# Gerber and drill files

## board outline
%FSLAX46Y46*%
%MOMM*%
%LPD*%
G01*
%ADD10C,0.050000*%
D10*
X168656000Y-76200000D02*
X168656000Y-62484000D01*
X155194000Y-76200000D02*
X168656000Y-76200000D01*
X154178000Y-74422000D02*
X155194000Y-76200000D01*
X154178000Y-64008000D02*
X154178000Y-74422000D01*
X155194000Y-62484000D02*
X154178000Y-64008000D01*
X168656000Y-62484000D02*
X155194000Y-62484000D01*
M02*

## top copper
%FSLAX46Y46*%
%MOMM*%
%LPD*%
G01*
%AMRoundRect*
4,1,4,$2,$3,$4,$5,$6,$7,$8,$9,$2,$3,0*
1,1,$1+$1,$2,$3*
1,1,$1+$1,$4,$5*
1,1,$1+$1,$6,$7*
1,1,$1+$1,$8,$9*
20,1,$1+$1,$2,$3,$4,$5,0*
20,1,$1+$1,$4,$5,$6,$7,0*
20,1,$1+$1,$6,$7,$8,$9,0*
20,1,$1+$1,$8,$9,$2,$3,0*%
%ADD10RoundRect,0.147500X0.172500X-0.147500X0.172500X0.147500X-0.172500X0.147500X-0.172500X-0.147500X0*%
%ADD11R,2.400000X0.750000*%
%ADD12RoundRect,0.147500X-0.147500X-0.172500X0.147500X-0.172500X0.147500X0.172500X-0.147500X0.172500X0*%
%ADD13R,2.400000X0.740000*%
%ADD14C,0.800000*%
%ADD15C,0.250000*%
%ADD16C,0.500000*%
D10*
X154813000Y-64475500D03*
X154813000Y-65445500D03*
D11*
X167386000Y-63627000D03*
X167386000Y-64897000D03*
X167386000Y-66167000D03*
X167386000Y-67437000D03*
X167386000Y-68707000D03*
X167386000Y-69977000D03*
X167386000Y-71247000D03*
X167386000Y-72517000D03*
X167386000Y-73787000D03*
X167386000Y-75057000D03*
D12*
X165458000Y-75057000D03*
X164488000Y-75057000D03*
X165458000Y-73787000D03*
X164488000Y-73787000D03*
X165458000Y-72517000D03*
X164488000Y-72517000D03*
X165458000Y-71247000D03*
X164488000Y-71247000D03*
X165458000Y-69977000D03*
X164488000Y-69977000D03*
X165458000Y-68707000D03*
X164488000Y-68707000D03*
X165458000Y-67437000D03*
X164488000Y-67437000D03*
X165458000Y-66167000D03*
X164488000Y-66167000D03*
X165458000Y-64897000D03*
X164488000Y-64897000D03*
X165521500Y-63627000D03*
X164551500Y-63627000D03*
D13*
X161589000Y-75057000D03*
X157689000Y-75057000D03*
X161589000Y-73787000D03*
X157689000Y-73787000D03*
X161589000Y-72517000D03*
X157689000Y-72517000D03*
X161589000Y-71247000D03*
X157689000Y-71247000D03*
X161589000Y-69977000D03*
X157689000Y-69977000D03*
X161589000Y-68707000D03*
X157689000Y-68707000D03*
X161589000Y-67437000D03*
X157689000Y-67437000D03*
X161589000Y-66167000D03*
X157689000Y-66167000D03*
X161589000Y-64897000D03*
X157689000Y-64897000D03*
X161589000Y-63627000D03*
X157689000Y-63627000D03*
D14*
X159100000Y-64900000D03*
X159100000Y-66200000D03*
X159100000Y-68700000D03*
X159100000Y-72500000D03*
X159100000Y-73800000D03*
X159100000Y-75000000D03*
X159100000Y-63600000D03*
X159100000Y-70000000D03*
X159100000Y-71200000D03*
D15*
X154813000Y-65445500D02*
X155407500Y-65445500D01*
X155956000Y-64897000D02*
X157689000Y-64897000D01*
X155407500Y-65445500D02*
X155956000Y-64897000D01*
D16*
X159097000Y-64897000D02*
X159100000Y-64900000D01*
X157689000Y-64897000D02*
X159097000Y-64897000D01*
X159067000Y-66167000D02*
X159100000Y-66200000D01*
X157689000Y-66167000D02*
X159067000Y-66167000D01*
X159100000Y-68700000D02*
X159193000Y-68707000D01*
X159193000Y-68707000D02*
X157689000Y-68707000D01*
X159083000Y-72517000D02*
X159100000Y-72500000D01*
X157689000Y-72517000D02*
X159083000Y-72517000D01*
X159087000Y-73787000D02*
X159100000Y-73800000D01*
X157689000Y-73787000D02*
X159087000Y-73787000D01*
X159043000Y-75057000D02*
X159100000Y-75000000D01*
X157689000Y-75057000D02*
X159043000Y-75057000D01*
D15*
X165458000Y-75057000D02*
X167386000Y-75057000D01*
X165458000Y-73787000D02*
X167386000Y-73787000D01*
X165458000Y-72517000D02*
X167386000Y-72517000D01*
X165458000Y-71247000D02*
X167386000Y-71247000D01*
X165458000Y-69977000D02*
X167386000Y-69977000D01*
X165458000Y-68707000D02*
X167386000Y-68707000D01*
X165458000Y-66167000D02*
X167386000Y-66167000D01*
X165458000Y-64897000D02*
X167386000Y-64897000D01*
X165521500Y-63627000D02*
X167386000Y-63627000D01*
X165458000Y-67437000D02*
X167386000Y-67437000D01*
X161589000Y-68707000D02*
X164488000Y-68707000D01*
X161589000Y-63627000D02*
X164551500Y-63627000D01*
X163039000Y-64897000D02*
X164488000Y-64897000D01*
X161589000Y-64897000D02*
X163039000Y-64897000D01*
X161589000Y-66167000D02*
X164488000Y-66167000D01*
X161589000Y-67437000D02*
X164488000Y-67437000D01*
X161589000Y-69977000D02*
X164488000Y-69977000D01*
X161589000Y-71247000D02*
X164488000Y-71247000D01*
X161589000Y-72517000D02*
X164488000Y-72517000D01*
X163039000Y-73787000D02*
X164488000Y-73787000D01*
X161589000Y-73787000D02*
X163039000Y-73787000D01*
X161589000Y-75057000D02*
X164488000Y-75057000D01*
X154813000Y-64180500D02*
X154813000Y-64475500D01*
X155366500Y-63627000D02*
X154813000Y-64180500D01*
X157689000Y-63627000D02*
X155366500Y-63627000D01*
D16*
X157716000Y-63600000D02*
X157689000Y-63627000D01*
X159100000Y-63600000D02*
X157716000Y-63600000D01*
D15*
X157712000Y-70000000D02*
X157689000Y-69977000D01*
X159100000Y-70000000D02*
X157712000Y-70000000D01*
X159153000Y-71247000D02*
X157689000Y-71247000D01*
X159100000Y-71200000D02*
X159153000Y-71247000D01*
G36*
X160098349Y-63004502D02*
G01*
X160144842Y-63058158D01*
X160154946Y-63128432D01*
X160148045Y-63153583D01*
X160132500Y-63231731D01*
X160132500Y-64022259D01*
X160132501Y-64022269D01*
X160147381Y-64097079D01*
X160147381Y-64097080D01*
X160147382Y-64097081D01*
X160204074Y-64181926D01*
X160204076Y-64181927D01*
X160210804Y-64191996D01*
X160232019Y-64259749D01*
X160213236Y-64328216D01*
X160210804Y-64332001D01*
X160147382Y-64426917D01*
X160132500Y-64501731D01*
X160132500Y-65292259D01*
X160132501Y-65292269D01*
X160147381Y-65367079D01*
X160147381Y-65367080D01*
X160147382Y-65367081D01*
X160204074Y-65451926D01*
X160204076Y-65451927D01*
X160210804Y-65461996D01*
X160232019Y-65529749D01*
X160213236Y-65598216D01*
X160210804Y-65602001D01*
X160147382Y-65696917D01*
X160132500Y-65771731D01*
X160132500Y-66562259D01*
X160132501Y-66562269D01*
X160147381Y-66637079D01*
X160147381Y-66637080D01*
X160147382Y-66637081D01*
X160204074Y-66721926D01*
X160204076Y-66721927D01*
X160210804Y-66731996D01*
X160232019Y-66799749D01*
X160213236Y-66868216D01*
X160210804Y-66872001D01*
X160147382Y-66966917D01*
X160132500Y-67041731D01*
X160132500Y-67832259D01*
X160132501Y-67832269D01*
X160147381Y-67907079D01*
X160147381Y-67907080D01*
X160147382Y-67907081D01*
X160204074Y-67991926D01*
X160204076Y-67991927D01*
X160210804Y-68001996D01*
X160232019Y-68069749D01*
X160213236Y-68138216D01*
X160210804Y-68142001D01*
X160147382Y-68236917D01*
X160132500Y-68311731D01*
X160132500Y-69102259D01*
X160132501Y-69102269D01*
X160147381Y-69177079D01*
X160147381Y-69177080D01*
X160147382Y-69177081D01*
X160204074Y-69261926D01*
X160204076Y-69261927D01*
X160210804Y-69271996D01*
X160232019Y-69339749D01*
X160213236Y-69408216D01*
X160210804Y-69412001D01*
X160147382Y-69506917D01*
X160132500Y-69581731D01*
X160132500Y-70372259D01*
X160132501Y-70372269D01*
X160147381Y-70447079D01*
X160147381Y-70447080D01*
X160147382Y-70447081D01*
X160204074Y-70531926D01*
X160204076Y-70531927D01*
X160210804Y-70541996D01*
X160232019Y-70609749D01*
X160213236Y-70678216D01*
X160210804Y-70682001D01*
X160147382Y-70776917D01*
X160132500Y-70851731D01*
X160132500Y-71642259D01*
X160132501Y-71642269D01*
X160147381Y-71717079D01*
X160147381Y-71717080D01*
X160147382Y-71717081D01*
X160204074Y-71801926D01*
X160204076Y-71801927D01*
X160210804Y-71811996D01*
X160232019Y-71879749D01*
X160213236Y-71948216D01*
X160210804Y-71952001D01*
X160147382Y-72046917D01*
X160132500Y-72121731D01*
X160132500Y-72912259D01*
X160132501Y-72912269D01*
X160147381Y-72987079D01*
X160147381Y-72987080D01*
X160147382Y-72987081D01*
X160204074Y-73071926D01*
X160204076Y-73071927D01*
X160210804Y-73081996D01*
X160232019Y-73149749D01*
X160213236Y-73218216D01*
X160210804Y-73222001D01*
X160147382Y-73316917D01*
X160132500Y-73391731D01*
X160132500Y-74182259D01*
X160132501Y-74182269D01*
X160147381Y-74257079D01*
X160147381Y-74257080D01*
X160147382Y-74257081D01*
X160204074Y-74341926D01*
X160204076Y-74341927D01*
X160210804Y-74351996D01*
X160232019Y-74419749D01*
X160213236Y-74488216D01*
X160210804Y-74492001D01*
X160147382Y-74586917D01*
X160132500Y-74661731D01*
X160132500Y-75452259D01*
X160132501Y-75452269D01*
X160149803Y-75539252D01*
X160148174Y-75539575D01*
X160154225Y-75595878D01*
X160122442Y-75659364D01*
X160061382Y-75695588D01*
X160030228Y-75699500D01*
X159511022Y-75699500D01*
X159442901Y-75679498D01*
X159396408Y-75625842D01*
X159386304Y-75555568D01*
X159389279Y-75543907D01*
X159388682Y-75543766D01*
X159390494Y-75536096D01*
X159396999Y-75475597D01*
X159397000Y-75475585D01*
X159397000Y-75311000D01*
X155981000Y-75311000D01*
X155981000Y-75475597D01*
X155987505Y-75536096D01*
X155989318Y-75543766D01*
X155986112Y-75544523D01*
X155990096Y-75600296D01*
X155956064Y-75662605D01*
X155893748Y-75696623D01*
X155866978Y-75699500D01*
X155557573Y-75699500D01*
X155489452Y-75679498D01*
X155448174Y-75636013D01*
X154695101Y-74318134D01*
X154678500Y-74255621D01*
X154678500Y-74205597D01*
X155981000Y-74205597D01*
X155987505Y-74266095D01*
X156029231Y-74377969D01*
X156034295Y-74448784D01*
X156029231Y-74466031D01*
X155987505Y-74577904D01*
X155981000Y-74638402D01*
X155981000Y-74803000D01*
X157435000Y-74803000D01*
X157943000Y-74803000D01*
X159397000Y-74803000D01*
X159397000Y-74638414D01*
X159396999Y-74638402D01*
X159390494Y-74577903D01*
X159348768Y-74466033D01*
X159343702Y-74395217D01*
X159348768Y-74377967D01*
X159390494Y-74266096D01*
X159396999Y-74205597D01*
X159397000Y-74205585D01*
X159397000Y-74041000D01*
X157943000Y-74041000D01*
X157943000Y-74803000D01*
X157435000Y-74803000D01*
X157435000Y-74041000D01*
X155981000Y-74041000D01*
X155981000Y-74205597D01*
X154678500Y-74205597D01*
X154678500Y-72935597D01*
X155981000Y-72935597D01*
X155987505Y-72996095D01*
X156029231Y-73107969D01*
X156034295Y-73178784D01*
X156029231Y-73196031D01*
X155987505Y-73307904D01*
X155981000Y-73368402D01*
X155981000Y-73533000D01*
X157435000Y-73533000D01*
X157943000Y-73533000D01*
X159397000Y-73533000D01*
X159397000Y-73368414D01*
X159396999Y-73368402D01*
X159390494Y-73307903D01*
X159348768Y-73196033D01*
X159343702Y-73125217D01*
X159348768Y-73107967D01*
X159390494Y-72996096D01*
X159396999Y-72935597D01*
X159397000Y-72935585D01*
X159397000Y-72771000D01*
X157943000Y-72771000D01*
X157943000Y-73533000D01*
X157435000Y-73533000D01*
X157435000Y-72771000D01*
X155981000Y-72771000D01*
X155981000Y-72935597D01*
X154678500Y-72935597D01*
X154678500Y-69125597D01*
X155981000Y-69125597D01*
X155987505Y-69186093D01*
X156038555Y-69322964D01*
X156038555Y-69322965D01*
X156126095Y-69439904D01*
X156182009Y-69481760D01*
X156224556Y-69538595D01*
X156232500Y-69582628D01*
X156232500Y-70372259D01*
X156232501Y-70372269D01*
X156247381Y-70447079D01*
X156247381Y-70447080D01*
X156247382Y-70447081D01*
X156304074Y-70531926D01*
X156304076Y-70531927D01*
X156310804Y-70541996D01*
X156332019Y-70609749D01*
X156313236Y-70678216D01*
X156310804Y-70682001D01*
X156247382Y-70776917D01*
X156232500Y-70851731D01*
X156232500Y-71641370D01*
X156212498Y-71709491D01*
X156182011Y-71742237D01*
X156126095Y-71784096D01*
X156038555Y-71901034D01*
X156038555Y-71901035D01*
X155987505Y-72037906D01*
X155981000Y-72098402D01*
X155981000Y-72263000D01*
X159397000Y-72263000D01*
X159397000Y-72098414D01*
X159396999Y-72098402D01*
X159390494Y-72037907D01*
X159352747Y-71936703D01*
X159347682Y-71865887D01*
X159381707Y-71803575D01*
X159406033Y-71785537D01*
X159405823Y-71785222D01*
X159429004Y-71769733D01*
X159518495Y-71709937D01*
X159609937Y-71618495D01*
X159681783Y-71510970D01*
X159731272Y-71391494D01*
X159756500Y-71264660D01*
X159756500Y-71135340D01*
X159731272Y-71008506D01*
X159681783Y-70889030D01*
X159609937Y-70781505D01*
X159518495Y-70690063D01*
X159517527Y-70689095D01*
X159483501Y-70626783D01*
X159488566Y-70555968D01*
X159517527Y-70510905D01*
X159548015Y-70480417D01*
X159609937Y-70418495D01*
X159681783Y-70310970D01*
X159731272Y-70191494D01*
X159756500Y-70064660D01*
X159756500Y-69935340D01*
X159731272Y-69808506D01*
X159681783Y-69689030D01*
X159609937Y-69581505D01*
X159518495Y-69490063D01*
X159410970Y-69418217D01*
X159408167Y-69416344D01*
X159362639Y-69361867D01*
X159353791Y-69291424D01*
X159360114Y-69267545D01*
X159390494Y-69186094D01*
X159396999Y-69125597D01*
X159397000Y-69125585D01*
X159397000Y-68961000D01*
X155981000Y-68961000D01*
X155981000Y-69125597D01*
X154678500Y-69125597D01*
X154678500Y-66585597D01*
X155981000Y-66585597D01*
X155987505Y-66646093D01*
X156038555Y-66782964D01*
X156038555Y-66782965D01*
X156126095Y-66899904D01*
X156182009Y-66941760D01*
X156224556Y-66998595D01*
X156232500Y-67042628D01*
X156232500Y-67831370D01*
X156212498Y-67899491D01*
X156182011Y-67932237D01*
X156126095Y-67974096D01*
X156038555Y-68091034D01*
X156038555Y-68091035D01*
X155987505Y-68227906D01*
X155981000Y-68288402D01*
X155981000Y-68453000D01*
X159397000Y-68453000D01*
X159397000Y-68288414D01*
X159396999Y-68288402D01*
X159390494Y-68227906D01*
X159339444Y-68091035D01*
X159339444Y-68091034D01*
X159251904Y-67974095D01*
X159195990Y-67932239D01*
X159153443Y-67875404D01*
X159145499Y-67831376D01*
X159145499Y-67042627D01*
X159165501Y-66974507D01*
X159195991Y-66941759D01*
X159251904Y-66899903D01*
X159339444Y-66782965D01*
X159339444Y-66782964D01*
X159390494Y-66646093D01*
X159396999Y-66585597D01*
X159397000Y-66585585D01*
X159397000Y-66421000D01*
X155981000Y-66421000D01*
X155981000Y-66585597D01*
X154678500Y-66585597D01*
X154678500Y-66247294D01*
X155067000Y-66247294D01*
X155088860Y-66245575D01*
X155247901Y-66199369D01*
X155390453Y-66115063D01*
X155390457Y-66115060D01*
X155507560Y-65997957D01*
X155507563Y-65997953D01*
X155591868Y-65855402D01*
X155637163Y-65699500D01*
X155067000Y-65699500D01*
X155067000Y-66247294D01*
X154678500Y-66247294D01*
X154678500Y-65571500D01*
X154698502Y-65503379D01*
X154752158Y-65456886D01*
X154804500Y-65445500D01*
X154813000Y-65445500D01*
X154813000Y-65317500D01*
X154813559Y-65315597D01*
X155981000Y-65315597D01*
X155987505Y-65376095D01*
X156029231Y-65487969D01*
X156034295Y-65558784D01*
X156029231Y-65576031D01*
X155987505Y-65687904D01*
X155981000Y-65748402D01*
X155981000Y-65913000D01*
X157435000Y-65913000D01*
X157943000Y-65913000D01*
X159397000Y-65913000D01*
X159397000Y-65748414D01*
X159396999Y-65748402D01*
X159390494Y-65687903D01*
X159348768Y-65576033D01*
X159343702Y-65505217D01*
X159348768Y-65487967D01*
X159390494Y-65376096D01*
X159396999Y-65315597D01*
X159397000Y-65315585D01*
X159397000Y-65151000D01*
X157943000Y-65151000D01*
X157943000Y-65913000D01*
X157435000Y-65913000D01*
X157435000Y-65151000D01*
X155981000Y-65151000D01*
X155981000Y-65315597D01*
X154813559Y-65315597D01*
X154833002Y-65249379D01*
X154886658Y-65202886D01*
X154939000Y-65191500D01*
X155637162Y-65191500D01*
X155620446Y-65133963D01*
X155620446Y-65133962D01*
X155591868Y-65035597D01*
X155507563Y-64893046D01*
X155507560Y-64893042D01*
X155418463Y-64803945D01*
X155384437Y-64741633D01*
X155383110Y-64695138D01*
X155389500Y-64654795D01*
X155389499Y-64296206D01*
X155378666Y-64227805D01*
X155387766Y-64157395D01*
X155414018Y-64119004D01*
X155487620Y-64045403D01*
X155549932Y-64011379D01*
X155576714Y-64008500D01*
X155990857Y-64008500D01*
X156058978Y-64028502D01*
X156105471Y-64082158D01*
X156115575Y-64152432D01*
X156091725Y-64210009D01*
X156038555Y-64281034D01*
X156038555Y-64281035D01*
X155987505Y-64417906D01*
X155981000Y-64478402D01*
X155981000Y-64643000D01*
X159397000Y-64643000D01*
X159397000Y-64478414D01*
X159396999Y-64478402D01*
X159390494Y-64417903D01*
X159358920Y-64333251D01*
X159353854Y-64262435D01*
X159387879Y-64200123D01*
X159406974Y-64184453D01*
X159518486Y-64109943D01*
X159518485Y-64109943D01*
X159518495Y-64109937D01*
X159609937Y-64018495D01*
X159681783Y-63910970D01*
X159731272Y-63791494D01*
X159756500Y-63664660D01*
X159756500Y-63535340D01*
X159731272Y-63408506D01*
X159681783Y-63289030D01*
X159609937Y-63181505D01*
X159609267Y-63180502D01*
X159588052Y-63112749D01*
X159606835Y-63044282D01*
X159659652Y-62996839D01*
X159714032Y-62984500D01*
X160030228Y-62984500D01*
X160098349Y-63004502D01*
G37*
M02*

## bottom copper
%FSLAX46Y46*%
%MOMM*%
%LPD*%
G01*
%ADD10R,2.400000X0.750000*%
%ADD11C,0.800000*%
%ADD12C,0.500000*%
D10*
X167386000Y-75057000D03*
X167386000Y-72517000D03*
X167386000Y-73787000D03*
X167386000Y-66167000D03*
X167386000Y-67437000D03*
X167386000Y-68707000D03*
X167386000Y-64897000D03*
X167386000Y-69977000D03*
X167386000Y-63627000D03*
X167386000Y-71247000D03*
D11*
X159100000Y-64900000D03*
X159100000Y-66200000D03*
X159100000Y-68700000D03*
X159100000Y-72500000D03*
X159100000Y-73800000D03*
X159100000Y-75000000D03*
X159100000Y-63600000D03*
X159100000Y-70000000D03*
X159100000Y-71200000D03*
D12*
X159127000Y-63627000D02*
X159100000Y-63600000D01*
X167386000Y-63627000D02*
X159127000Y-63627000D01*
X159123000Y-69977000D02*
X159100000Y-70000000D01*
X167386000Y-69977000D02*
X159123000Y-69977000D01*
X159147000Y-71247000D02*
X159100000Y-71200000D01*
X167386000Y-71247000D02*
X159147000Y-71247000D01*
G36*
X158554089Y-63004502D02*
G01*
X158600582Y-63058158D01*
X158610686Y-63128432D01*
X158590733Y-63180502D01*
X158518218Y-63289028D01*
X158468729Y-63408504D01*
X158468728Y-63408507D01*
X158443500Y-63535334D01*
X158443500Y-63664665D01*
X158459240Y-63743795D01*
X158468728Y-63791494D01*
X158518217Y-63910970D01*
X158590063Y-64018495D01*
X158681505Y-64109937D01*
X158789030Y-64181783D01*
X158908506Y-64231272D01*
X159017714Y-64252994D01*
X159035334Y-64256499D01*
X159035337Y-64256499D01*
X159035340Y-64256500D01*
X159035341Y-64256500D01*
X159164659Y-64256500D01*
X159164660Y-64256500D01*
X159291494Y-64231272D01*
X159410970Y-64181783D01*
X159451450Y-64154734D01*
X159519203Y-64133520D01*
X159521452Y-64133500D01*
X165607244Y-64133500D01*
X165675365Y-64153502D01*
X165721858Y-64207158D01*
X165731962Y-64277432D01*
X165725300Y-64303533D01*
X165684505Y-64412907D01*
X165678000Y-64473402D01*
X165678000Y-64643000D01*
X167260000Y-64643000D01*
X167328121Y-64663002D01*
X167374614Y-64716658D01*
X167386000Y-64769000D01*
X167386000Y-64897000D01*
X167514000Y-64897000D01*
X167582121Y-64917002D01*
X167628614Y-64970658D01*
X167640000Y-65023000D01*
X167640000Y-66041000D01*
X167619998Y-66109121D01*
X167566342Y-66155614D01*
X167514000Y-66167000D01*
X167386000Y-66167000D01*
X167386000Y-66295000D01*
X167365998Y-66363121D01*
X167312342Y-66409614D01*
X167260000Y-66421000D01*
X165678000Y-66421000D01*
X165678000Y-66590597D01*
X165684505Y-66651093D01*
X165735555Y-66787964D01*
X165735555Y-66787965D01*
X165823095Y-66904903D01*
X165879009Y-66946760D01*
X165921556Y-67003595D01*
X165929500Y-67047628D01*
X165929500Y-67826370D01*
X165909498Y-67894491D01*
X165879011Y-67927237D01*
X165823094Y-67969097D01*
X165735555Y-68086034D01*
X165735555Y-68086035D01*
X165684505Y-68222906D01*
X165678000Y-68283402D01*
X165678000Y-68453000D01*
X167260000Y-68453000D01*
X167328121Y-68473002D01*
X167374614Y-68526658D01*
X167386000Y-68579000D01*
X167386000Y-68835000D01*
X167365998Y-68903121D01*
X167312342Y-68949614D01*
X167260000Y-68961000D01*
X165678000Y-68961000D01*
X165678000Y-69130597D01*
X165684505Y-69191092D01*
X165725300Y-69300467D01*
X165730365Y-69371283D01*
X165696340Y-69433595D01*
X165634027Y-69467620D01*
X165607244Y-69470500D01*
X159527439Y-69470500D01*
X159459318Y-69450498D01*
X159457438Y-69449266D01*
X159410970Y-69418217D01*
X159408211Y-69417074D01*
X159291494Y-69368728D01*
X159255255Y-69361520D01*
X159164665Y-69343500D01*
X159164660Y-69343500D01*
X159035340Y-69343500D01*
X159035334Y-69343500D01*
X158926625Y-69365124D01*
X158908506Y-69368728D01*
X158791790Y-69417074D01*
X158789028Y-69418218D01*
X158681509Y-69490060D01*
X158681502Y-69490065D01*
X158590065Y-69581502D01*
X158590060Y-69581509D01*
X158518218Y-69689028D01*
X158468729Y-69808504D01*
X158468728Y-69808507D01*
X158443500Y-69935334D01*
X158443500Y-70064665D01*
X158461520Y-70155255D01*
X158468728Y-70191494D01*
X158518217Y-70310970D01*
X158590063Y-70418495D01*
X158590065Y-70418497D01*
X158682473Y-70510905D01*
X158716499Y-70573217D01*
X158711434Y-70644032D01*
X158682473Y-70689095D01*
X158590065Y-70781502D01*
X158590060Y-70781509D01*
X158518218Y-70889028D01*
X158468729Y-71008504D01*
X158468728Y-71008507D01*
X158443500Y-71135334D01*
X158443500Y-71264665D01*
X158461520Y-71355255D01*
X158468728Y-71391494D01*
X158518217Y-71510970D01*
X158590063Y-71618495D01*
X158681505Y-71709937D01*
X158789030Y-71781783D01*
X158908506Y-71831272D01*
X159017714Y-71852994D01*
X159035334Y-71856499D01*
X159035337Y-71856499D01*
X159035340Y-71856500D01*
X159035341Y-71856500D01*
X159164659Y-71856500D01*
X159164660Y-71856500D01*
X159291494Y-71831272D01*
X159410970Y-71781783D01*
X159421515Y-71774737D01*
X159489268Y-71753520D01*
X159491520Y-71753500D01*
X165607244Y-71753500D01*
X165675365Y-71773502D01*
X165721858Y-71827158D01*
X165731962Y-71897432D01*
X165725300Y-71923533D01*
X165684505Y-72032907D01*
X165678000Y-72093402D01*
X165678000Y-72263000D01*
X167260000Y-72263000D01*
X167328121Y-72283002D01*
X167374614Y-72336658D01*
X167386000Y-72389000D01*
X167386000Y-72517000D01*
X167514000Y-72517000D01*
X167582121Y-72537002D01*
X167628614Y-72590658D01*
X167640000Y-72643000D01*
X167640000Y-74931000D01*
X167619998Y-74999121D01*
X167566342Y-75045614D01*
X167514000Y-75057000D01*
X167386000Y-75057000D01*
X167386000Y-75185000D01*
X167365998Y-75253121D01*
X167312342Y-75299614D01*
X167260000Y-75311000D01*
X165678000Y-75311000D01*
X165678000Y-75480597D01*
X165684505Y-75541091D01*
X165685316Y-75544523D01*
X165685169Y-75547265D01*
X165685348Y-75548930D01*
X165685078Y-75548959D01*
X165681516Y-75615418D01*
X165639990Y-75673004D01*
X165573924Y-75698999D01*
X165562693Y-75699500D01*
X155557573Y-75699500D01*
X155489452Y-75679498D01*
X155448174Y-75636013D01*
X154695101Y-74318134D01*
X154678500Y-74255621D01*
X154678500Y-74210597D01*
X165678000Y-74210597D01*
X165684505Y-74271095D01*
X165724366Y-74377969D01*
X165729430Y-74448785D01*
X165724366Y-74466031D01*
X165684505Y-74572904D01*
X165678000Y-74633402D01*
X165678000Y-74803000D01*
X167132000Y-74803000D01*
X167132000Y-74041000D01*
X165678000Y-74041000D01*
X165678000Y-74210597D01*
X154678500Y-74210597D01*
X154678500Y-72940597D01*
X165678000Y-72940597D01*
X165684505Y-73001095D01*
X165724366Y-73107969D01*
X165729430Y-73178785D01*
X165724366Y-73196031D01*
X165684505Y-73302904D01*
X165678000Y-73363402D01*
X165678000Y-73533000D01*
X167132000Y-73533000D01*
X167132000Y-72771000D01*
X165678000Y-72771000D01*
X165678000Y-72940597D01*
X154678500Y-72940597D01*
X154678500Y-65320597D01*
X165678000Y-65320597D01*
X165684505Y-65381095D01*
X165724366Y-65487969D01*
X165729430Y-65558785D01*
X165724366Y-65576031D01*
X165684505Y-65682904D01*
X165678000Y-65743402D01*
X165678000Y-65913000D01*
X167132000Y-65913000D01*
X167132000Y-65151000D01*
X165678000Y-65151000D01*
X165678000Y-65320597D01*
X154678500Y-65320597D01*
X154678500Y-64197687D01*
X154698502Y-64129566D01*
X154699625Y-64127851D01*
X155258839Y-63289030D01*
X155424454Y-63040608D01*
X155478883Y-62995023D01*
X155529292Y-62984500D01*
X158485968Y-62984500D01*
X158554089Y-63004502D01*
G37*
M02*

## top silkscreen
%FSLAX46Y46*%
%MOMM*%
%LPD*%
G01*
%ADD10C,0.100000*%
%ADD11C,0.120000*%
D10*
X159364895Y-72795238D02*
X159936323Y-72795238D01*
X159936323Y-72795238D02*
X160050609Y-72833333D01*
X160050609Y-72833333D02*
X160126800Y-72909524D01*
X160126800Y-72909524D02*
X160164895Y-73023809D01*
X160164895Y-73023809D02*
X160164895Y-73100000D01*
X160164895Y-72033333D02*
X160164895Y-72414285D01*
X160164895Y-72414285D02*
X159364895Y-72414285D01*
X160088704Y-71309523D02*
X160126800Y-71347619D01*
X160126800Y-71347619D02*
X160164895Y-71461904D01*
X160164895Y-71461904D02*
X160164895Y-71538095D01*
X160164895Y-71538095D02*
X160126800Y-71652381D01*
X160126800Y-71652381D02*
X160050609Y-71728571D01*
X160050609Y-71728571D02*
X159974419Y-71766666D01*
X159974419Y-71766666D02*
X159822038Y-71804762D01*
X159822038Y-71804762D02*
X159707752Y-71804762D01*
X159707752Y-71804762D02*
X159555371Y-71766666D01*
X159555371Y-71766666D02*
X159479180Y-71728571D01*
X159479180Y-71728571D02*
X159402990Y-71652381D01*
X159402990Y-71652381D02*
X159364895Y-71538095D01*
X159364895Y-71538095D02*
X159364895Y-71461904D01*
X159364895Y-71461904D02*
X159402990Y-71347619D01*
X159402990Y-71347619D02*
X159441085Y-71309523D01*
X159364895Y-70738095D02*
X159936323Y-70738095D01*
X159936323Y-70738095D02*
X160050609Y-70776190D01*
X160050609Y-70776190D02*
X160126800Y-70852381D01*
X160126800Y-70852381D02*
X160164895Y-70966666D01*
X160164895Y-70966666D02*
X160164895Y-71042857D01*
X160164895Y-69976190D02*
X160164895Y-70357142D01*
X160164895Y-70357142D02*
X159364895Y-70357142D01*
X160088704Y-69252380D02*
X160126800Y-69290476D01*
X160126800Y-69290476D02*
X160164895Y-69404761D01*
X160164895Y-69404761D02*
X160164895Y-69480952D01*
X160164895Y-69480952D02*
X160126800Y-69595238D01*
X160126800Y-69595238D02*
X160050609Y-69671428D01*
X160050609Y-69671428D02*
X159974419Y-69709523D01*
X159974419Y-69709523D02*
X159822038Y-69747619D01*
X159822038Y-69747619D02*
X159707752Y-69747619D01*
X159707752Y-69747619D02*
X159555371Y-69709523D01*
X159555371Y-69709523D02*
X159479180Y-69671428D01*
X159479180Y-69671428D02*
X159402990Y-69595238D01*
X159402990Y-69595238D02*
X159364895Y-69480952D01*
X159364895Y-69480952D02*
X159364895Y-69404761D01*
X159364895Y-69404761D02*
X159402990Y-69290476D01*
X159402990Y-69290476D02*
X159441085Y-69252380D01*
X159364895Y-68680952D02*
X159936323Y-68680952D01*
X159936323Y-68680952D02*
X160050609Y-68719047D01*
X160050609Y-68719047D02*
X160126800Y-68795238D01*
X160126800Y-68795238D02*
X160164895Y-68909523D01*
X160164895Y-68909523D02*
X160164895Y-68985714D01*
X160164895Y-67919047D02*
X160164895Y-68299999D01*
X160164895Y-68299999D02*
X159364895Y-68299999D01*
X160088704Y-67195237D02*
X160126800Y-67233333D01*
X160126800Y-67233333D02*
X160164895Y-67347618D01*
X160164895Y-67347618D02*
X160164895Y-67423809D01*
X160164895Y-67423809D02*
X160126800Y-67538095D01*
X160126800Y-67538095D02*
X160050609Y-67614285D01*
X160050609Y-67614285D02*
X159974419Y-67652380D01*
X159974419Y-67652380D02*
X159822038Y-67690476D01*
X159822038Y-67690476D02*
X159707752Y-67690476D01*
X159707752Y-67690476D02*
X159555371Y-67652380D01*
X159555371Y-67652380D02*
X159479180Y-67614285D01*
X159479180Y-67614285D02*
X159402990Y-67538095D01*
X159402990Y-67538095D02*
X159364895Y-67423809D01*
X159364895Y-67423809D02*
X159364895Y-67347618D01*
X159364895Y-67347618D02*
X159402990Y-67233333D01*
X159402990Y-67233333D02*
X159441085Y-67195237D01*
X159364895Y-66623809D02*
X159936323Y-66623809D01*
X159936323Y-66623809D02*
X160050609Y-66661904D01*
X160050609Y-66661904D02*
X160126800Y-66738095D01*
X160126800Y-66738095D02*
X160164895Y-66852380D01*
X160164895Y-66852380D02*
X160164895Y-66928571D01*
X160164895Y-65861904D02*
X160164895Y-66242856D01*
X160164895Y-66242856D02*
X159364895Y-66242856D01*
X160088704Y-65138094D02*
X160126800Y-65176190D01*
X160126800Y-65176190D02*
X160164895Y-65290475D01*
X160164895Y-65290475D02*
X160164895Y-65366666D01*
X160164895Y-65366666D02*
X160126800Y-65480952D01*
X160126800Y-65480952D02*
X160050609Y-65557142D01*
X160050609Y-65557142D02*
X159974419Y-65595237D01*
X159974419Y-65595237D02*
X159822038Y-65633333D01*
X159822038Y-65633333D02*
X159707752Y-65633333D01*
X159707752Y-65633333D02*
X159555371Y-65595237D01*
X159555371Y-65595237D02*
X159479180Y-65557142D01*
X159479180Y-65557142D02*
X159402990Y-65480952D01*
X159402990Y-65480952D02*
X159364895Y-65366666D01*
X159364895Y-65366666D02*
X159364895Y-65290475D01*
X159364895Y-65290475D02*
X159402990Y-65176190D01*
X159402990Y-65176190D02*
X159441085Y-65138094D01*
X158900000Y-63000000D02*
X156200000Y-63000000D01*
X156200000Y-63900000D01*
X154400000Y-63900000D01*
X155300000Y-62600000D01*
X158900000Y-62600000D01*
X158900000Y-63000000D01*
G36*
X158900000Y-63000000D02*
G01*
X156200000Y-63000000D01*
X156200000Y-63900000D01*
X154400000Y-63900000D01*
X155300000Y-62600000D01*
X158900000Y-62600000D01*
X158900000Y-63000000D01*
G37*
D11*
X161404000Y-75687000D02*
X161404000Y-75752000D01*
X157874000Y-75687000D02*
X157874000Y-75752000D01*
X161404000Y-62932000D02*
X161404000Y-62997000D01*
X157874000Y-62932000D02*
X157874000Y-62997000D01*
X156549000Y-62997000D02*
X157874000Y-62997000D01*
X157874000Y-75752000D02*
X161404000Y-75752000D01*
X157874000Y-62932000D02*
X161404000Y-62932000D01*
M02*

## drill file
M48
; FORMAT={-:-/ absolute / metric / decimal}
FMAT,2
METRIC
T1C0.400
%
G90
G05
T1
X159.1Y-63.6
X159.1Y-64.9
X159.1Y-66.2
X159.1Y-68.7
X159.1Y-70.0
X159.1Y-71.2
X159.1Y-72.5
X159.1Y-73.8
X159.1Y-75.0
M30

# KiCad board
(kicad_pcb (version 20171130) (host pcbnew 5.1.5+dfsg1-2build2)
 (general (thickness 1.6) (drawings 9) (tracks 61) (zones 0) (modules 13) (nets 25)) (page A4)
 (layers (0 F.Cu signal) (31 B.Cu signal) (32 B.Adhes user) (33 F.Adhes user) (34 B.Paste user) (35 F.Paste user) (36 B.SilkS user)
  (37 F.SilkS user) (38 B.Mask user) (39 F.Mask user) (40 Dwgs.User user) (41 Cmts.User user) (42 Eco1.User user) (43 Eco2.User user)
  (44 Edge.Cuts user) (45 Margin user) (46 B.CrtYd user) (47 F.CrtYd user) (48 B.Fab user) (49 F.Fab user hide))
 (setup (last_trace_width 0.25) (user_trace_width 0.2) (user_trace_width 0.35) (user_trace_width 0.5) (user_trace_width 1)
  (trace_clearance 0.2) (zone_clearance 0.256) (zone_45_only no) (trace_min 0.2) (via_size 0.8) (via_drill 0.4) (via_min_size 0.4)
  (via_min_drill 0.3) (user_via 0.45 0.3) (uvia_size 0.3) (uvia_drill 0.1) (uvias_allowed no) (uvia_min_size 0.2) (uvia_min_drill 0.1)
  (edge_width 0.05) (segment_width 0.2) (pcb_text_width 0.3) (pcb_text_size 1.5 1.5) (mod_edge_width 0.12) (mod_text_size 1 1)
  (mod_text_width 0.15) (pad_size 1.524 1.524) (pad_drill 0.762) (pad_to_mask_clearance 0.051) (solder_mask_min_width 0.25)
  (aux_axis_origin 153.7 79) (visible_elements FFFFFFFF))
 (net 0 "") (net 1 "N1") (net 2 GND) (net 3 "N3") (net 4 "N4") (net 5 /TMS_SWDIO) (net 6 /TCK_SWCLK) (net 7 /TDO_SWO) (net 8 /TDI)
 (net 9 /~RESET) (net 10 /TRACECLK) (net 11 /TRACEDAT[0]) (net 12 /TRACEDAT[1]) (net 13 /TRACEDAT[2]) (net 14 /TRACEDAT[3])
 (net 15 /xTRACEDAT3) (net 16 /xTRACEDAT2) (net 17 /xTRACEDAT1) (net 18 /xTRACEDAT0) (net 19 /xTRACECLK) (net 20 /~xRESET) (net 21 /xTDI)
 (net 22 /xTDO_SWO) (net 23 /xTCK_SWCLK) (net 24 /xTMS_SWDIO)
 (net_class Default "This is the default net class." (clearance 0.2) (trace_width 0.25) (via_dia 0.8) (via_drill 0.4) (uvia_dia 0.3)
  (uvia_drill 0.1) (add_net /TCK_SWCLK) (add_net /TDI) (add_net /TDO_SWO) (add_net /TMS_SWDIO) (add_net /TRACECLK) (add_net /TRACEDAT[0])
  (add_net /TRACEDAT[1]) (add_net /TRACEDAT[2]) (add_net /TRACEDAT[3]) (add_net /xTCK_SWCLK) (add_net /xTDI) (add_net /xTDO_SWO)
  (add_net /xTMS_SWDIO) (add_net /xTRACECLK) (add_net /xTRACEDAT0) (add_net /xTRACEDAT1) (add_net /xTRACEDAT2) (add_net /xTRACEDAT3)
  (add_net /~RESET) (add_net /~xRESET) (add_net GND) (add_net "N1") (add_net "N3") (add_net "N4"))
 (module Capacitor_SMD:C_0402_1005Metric (layer F.Cu) (at 154.813 64.9605 90)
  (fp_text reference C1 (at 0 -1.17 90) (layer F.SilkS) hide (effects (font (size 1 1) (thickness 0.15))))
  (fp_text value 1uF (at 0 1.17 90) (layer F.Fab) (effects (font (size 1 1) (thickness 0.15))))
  (pad 2 smd roundrect (at 0.485 0 90) (size 0.59 0.64) (layers F.Cu F.Paste F.Mask) (roundrect_rratio 0.25) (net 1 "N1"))
  (pad 1 smd roundrect (at -0.485 0 90) (size 0.59 0.64) (layers F.Cu F.Paste F.Mask) (roundrect_rratio 0.25) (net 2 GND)))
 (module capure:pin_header (layer F.Cu) (at 167.386 75.057)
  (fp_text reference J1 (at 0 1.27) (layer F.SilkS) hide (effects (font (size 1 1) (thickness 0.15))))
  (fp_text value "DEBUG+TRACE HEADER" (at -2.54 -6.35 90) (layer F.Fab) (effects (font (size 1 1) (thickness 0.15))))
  (pad 19 smd rect (at 0 0) (size 2.4 0.75) (layers B.Cu B.Paste B.Mask) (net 2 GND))
  (pad 15 smd rect (at 0 -2.54) (size 2.4 0.75) (layers B.Cu B.Paste B.Mask) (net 2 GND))
  (pad 17 smd rect (at 0 -1.27) (size 2.4 0.75) (layers B.Cu B.Paste B.Mask) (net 2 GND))
  (pad 5 smd rect (at 0 -8.89) (size 2.4 0.75) (layers B.Cu B.Paste B.Mask) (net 2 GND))
  (pad 7 smd rect (at 0 -7.62) (size 2.4 0.75) (layers B.Cu B.Paste B.Mask))
  (pad 9 smd rect (at 0 -6.35) (size 2.4 0.75) (layers B.Cu B.Paste B.Mask) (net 2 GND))
  (pad 3 smd rect (at 0 -10.16) (size 2.4 0.75) (layers B.Cu B.Paste B.Mask) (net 2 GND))
  (pad 11 smd rect (at 0 -5.08) (size 2.4 0.75) (layers B.Cu B.Paste B.Mask) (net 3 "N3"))
  (pad 1 smd rect (at 0 -11.43) (size 2.4 0.75) (layers B.Cu B.Paste B.Mask) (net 1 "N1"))
  (pad 13 smd rect (at 0 -3.81) (size 2.4 0.75) (layers B.Cu B.Paste B.Mask) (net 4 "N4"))
  (pad 2 smd rect (at 0 -11.43) (size 2.4 0.75) (layers F.Cu F.Paste F.Mask) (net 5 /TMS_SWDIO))
  (pad 4 smd rect (at 0 -10.16) (size 2.4 0.75) (layers F.Cu F.Paste F.Mask) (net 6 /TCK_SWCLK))
  (pad 6 smd rect (at 0 -8.89) (size 2.4 0.75) (layers F.Cu F.Paste F.Mask) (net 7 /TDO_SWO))
  (pad 8 smd rect (at 0 -7.62) (size 2.4 0.75) (layers F.Cu F.Paste F.Mask) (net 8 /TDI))
  (pad 10 smd rect (at 0 -6.35) (size 2.4 0.75) (layers F.Cu F.Paste F.Mask) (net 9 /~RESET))
  (pad 12 smd rect (at 0 -5.08) (size 2.4 0.75) (layers F.Cu F.Paste F.Mask) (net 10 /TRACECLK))
  (pad 14 smd rect (at 0 -3.81) (size 2.4 0.75) (layers F.Cu F.Paste F.Mask) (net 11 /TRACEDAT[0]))
  (pad 16 smd rect (at 0 -2.54) (size 2.4 0.75) (layers F.Cu F.Paste F.Mask) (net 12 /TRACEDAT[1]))
  (pad 18 smd rect (at 0 -1.27) (size 2.4 0.75) (layers F.Cu F.Paste F.Mask) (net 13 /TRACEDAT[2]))
  (pad 20 smd rect (at 0 0) (size 2.4 0.75) (layers F.Cu F.Paste F.Mask) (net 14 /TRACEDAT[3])))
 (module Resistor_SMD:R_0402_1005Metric (layer F.Cu) (at 164.973 75.057)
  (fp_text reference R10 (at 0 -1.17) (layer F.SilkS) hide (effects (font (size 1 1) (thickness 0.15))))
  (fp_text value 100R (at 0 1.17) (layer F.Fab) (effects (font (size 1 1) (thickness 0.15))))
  (pad 2 smd roundrect (at 0.485 0) (size 0.59 0.64) (layers F.Cu F.Paste F.Mask) (roundrect_rratio 0.25) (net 14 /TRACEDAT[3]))
  (pad 1 smd roundrect (at -0.485 0) (size 0.59 0.64) (layers F.Cu F.Paste F.Mask) (roundrect_rratio 0.25) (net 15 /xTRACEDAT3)))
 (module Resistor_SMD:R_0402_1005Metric (layer F.Cu) (at 164.973 73.787)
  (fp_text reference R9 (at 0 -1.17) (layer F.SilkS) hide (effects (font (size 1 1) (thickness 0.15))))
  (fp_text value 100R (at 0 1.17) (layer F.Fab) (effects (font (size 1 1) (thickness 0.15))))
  (pad 2 smd roundrect (at 0.485 0) (size 0.59 0.64) (layers F.Cu F.Paste F.Mask) (roundrect_rratio 0.25) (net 13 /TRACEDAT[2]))
  (pad 1 smd roundrect (at -0.485 0) (size 0.59 0.64) (layers F.Cu F.Paste F.Mask) (roundrect_rratio 0.25) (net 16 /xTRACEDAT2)))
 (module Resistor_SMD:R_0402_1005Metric (layer F.Cu) (at 164.973 72.517)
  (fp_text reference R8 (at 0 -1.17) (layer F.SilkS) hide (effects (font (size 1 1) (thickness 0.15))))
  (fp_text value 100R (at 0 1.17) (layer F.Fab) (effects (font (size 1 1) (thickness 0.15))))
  (pad 2 smd roundrect (at 0.485 0) (size 0.59 0.64) (layers F.Cu F.Paste F.Mask) (roundrect_rratio 0.25) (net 12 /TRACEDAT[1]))
  (pad 1 smd roundrect (at -0.485 0) (size 0.59 0.64) (layers F.Cu F.Paste F.Mask) (roundrect_rratio 0.25) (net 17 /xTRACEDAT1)))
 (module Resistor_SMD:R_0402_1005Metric (layer F.Cu) (at 164.973 71.247)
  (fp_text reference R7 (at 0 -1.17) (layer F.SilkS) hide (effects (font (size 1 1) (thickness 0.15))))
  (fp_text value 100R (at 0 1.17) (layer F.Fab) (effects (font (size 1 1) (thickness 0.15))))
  (pad 2 smd roundrect (at 0.485 0) (size 0.59 0.64) (layers F.Cu F.Paste F.Mask) (roundrect_rratio 0.25) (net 11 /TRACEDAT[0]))
  (pad 1 smd roundrect (at -0.485 0) (size 0.59 0.64) (layers F.Cu F.Paste F.Mask) (roundrect_rratio 0.25) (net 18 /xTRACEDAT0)))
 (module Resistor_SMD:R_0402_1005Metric (layer F.Cu) (at 164.973 69.977)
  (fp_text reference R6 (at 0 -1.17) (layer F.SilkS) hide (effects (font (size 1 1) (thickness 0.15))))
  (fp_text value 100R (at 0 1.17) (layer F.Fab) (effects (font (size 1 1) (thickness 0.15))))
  (pad 2 smd roundrect (at 0.485 0) (size 0.59 0.64) (layers F.Cu F.Paste F.Mask) (roundrect_rratio 0.25) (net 10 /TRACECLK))
  (pad 1 smd roundrect (at -0.485 0) (size 0.59 0.64) (layers F.Cu F.Paste F.Mask) (roundrect_rratio 0.25) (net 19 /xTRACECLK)))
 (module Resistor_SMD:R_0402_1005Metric (layer F.Cu) (at 164.973 68.707)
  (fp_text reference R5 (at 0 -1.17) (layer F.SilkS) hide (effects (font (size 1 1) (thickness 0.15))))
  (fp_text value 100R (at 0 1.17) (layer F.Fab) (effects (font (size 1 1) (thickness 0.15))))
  (pad 2 smd roundrect (at 0.485 0) (size 0.59 0.64) (layers F.Cu F.Paste F.Mask) (roundrect_rratio 0.25) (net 9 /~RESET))
  (pad 1 smd roundrect (at -0.485 0) (size 0.59 0.64) (layers F.Cu F.Paste F.Mask) (roundrect_rratio 0.25) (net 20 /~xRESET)))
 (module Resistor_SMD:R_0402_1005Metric (layer F.Cu) (at 164.973 67.437)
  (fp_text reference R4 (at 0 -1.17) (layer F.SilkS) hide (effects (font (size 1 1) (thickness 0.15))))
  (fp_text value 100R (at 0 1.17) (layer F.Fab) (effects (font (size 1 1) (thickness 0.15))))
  (pad 2 smd roundrect (at 0.485 0) (size 0.59 0.64) (layers F.Cu F.Paste F.Mask) (roundrect_rratio 0.25) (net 8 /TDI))
  (pad 1 smd roundrect (at -0.485 0) (size 0.59 0.64) (layers F.Cu F.Paste F.Mask) (roundrect_rratio 0.25) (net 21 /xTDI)))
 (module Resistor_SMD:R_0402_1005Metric (layer F.Cu) (at 164.973 66.167)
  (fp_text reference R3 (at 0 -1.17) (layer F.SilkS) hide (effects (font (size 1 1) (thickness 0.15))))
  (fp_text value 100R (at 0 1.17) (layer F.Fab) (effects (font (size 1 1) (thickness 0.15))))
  (pad 2 smd roundrect (at 0.485 0) (size 0.59 0.64) (layers F.Cu F.Paste F.Mask) (roundrect_rratio 0.25) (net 7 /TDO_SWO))
  (pad 1 smd roundrect (at -0.485 0) (size 0.59 0.64) (layers F.Cu F.Paste F.Mask) (roundrect_rratio 0.25) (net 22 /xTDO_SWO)))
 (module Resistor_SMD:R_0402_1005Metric (layer F.Cu) (at 164.973 64.897)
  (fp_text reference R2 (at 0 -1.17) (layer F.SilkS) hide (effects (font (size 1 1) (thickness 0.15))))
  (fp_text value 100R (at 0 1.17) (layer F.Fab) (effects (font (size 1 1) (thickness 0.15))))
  (pad 2 smd roundrect (at 0.485 0) (size 0.59 0.64) (layers F.Cu F.Paste F.Mask) (roundrect_rratio 0.25) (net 6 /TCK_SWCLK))
  (pad 1 smd roundrect (at -0.485 0) (size 0.59 0.64) (layers F.Cu F.Paste F.Mask) (roundrect_rratio 0.25) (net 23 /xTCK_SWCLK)))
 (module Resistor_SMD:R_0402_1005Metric (layer F.Cu) (at 165.0365 63.627)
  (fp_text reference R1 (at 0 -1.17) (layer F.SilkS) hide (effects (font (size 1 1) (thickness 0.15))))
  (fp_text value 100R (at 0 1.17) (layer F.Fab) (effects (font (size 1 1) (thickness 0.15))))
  (pad 2 smd roundrect (at 0.485 0) (size 0.59 0.64) (layers F.Cu F.Paste F.Mask) (roundrect_rratio 0.25) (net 5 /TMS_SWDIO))
  (pad 1 smd roundrect (at -0.485 0) (size 0.59 0.64) (layers F.Cu F.Paste F.Mask) (roundrect_rratio 0.25) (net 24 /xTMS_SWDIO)))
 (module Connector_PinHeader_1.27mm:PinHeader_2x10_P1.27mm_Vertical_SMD (layer F.Cu) (at 159.639 69.342)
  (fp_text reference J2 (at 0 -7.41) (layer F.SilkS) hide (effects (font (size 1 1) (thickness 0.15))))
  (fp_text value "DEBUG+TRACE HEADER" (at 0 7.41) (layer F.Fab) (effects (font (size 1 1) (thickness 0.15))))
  (fp_line (start 1.765 6.345) (end 1.765 6.41) (layer F.SilkS) (width 0.12))
  (fp_line (start -1.765 6.345) (end -1.765 6.41) (layer F.SilkS) (width 0.12))
  (fp_line (start 1.765 -6.41) (end 1.765 -6.345) (layer F.SilkS) (width 0.12))
  (fp_line (start -1.765 -6.41) (end -1.765 -6.345) (layer F.SilkS) (width 0.12))
  (fp_line (start -3.09 -6.345) (end -1.765 -6.345) (layer F.SilkS) (width 0.12))
  (fp_line (start -1.765 6.41) (end 1.765 6.41) (layer F.SilkS) (width 0.12))
  (fp_line (start -1.765 -6.41) (end 1.765 -6.41) (layer F.SilkS) (width 0.12))
  (pad 20 smd rect (at 1.95 5.715) (size 2.4 0.74) (layers F.Cu F.Paste F.Mask) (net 15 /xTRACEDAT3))
  (pad 19 smd rect (at -1.95 5.715) (size 2.4 0.74) (layers F.Cu F.Paste F.Mask) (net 2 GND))
  (pad 18 smd rect (at 1.95 4.445) (size 2.4 0.74) (layers F.Cu F.Paste F.Mask) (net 16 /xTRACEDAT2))
  (pad 17 smd rect (at -1.95 4.445) (size 2.4 0.74) (layers F.Cu F.Paste F.Mask) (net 2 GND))
  (pad 16 smd rect (at 1.95 3.175) (size 2.4 0.74) (layers F.Cu F.Paste F.Mask) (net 17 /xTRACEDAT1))
  (pad 15 smd rect (at -1.95 3.175) (size 2.4 0.74) (layers F.Cu F.Paste F.Mask) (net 2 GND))
  (pad 14 smd rect (at 1.95 1.905) (size 2.4 0.74) (layers F.Cu F.Paste F.Mask) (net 18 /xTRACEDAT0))
  (pad 13 smd rect (at -1.95 1.905) (size 2.4 0.74) (layers F.Cu F.Paste F.Mask) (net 4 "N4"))
  (pad 12 smd rect (at 1.95 0.635) (size 2.4 0.74) (layers F.Cu F.Paste F.Mask) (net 19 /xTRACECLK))
  (pad 11 smd rect (at -1.95 0.635) (size 2.4 0.74) (layers F.Cu F.Paste F.Mask) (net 3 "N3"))
  (pad 10 smd rect (at 1.95 -0.635) (size 2.4 0.74) (layers F.Cu F.Paste F.Mask) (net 20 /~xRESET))
  (pad 9 smd rect (at -1.95 -0.635) (size 2.4 0.74) (layers F.Cu F.Paste F.Mask) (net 2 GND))
  (pad 8 smd rect (at 1.95 -1.905) (size 2.4 0.74) (layers F.Cu F.Paste F.Mask) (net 21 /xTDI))
  (pad 7 smd rect (at -1.95 -1.905) (size 2.4 0.74) (layers F.Cu F.Paste F.Mask))
  (pad 6 smd rect (at 1.95 -3.175) (size 2.4 0.74) (layers F.Cu F.Paste F.Mask) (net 22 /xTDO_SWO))
  (pad 5 smd rect (at -1.95 -3.175) (size 2.4 0.74) (layers F.Cu F.Paste F.Mask) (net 2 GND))
  (pad 4 smd rect (at 1.95 -4.445) (size 2.4 0.74) (layers F.Cu F.Paste F.Mask) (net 23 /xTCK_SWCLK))
  (pad 3 smd rect (at -1.95 -4.445) (size 2.4 0.74) (layers F.Cu F.Paste F.Mask) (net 2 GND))
  (pad 2 smd rect (at 1.95 -5.715) (size 2.4 0.74) (layers F.Cu F.Paste F.Mask) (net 24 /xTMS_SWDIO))
  (pad 1 smd rect (at -1.95 -5.715) (size 2.4 0.74) (layers F.Cu F.Paste F.Mask) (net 1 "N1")))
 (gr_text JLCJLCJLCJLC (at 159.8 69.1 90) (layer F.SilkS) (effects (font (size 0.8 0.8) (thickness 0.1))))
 (gr_poly (pts (xy 158.9 63) (xy 156.2 63) (xy 156.2 63.9) (xy 154.4 63.9) (xy 155.3 62.6) (xy 158.9 62.6)) (layer F.SilkS) (width 0.1))
 (gr_line (start 168.656 76.2) (end 168.656 62.484) (layer Edge.Cuts) (width 0.05))
 (gr_line (start 155.194 76.2) (end 168.656 76.2) (layer Edge.Cuts) (width 0.05))
 (gr_line (start 154.178 74.422) (end 155.194 76.2) (layer Edge.Cuts) (width 0.05))
 (gr_line (start 154.178 64.008) (end 154.178 74.422) (layer Edge.Cuts) (width 0.05))
 (gr_line (start 155.194 62.484) (end 154.178 64.008) (layer Edge.Cuts) (width 0.05))
 (gr_line (start 168.656 62.484) (end 155.194 62.484) (layer Edge.Cuts) (width 0.05))
 (segment (start 154.813 65.4455) (end 155.4075 65.4455) (width 0.25) (layer F.Cu) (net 2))
 (segment (start 155.956 64.897) (end 157.689 64.897) (width 0.25) (layer F.Cu) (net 2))
 (segment (start 155.4075 65.4455) (end 155.956 64.897) (width 0.25) (layer F.Cu) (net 2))
 (via (at 159.1 64.9) (size 0.8) (drill 0.4) (layers F.Cu B.Cu) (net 2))
 (segment (start 159.097 64.897) (end 159.1 64.9) (width 0.5) (layer F.Cu) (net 2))
 (segment (start 157.689 64.897) (end 159.097 64.897) (width 0.5) (layer F.Cu) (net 2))
 (via (at 159.1 66.2) (size 0.8) (drill 0.4) (layers F.Cu B.Cu) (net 2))
 (segment (start 159.067 66.167) (end 159.1 66.2) (width 0.5) (layer F.Cu) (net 2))
 (segment (start 157.689 66.167) (end 159.067 66.167) (width 0.5) (layer F.Cu) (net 2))
 (segment (start 159.1 68.7) (end 159.193 68.707) (width 0.5) (layer F.Cu) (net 2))
 (segment (start 159.193 68.707) (end 157.689 68.707) (width 0.5) (layer F.Cu) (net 2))
 (via (at 159.1 68.7) (size 0.8) (drill 0.4) (layers F.Cu B.Cu) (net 2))
 (via (at 159.1 72.5) (size 0.8) (drill 0.4) (layers F.Cu B.Cu) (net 2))
 (segment (start 159.083 72.517) (end 159.1 72.5) (width 0.5) (layer F.Cu) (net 2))
 (segment (start 157.689 72.517) (end 159.083 72.517) (width 0.5) (layer F.Cu) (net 2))
 (via (at 159.1 73.8) (size 0.8) (drill 0.4) (layers F.Cu B.Cu) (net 2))
 (segment (start 159.087 73.787) (end 159.1 73.8) (width 0.5) (layer F.Cu) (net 2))
 (segment (start 157.689 73.787) (end 159.087 73.787) (width 0.5) (layer F.Cu) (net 2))
 (via (at 159.1 75) (size 0.8) (drill 0.4) (layers F.Cu B.Cu) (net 2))
 (segment (start 159.043 75.057) (end 159.1 75) (width 0.5) (layer F.Cu) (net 2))
 (segment (start 157.689 75.057) (end 159.043 75.057) (width 0.5) (layer F.Cu) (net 2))
 (segment (start 165.458 75.057) (end 167.386 75.057) (width 0.25) (layer F.Cu) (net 14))
 (segment (start 165.458 73.787) (end 167.386 73.787) (width 0.25) (layer F.Cu) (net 13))
 (segment (start 165.458 72.517) (end 167.386 72.517) (width 0.25) (layer F.Cu) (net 12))
 (segment (start 165.458 71.247) (end 167.386 71.247) (width 0.25) (layer F.Cu) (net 11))
 (segment (start 165.458 69.977) (end 167.386 69.977) (width 0.25) (layer F.Cu) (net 10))
 (segment (start 165.458 68.707) (end 167.386 68.707) (width 0.25) (layer F.Cu) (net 9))
 (segment (start 165.458 66.167) (end 167.386 66.167) (width 0.25) (layer F.Cu) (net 7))
 (segment (start 165.458 64.897) (end 167.386 64.897) (width 0.25) (layer F.Cu) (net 6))
 (segment (start 165.5215 63.627) (end 167.386 63.627) (width 0.25) (layer F.Cu) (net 5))
 (segment (start 165.458 67.437) (end 167.386 67.437) (width 0.25) (layer F.Cu) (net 8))
 (segment (start 161.589 68.707) (end 164.488 68.707) (width 0.25) (layer F.Cu) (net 20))
 (segment (start 161.589 63.627) (end 164.5515 63.627) (width 0.25) (layer F.Cu) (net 24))
 (segment (start 163.039 64.897) (end 164.488 64.897) (width 0.25) (layer F.Cu) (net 23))
 (segment (start 161.589 64.897) (end 163.039 64.897) (width 0.25) (layer F.Cu) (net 23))
 (segment (start 161.589 66.167) (end 164.488 66.167) (width 0.25) (layer F.Cu) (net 22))
 (segment (start 161.589 67.437) (end 164.488 67.437) (width 0.25) (layer F.Cu) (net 21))
 (segment (start 161.589 69.977) (end 164.488 69.977) (width 0.25) (layer F.Cu) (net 19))
 (segment (start 161.589 71.247) (end 164.488 71.247) (width 0.25) (layer F.Cu) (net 18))
 (segment (start 161.589 72.517) (end 164.488 72.517) (width 0.25) (layer F.Cu) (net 17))
 (segment (start 163.039 73.787) (end 164.488 73.787) (width 0.25) (layer F.Cu) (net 16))
 (segment (start 161.589 73.787) (end 163.039 73.787) (width 0.25) (layer F.Cu) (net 16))
 (segment (start 161.589 75.057) (end 164.488 75.057) (width 0.25) (layer F.Cu) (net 15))
 (segment (start 154.813 64.1805) (end 154.813 64.4755) (width 0.25) (layer F.Cu) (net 1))
 (segment (start 155.3665 63.627) (end 154.813 64.1805) (width 0.25) (layer F.Cu) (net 1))
 (segment (start 157.689 63.627) (end 155.3665 63.627) (width 0.25) (layer F.Cu) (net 1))
 (via (at 159.1 63.6) (size 0.8) (drill 0.4) (layers F.Cu B.Cu) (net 1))
 (segment (start 159.127 63.627) (end 159.1 63.6) (width 0.5) (layer B.Cu) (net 1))
 (segment (start 167.386 63.627) (end 159.127 63.627) (width 0.5) (layer B.Cu) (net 1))
 (segment (start 157.716 63.6) (end 157.689 63.627) (width 0.5) (layer F.Cu) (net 1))
 (segment (start 159.1 63.6) (end 157.716 63.6) (width 0.5) (layer F.Cu) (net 1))
 (via (at 159.1 70) (size 0.8) (drill 0.4) (layers F.Cu B.Cu) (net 3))
 (segment (start 157.712 70) (end 157.689 69.977) (width 0.25) (layer F.Cu) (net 3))
 (segment (start 159.1 70) (end 157.712 70) (width 0.25) (layer F.Cu) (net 3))
 (segment (start 159.123 69.977) (end 159.1 70) (width 0.5) (layer B.Cu) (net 3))
 (segment (start 167.386 69.977) (end 159.123 69.977) (width 0.5) (layer B.Cu) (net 3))
 (segment (start 159.153 71.247) (end 157.689 71.247) (width 0.25) (layer F.Cu) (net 4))
 (segment (start 159.1 71.2) (end 159.153 71.247) (width 0.25) (layer F.Cu) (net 4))
 (via (at 159.1 71.2) (size 0.8) (drill 0.4) (layers F.Cu B.Cu) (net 4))
 (segment (start 159.147 71.247) (end 159.1 71.2) (width 0.5) (layer B.Cu) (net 4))
 (segment (start 167.386 71.247) (end 159.147 71.247) (width 0.5) (layer B.Cu) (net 4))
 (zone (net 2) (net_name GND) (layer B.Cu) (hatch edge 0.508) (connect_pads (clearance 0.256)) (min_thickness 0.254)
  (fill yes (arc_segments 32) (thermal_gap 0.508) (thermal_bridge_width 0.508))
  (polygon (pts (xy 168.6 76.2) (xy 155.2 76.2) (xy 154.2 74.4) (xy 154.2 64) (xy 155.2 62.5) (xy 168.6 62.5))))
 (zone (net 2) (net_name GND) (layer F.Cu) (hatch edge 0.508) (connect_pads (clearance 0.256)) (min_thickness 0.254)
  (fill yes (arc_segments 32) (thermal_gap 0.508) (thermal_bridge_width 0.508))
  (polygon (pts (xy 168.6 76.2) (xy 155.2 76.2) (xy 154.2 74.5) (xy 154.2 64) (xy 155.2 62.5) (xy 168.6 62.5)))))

